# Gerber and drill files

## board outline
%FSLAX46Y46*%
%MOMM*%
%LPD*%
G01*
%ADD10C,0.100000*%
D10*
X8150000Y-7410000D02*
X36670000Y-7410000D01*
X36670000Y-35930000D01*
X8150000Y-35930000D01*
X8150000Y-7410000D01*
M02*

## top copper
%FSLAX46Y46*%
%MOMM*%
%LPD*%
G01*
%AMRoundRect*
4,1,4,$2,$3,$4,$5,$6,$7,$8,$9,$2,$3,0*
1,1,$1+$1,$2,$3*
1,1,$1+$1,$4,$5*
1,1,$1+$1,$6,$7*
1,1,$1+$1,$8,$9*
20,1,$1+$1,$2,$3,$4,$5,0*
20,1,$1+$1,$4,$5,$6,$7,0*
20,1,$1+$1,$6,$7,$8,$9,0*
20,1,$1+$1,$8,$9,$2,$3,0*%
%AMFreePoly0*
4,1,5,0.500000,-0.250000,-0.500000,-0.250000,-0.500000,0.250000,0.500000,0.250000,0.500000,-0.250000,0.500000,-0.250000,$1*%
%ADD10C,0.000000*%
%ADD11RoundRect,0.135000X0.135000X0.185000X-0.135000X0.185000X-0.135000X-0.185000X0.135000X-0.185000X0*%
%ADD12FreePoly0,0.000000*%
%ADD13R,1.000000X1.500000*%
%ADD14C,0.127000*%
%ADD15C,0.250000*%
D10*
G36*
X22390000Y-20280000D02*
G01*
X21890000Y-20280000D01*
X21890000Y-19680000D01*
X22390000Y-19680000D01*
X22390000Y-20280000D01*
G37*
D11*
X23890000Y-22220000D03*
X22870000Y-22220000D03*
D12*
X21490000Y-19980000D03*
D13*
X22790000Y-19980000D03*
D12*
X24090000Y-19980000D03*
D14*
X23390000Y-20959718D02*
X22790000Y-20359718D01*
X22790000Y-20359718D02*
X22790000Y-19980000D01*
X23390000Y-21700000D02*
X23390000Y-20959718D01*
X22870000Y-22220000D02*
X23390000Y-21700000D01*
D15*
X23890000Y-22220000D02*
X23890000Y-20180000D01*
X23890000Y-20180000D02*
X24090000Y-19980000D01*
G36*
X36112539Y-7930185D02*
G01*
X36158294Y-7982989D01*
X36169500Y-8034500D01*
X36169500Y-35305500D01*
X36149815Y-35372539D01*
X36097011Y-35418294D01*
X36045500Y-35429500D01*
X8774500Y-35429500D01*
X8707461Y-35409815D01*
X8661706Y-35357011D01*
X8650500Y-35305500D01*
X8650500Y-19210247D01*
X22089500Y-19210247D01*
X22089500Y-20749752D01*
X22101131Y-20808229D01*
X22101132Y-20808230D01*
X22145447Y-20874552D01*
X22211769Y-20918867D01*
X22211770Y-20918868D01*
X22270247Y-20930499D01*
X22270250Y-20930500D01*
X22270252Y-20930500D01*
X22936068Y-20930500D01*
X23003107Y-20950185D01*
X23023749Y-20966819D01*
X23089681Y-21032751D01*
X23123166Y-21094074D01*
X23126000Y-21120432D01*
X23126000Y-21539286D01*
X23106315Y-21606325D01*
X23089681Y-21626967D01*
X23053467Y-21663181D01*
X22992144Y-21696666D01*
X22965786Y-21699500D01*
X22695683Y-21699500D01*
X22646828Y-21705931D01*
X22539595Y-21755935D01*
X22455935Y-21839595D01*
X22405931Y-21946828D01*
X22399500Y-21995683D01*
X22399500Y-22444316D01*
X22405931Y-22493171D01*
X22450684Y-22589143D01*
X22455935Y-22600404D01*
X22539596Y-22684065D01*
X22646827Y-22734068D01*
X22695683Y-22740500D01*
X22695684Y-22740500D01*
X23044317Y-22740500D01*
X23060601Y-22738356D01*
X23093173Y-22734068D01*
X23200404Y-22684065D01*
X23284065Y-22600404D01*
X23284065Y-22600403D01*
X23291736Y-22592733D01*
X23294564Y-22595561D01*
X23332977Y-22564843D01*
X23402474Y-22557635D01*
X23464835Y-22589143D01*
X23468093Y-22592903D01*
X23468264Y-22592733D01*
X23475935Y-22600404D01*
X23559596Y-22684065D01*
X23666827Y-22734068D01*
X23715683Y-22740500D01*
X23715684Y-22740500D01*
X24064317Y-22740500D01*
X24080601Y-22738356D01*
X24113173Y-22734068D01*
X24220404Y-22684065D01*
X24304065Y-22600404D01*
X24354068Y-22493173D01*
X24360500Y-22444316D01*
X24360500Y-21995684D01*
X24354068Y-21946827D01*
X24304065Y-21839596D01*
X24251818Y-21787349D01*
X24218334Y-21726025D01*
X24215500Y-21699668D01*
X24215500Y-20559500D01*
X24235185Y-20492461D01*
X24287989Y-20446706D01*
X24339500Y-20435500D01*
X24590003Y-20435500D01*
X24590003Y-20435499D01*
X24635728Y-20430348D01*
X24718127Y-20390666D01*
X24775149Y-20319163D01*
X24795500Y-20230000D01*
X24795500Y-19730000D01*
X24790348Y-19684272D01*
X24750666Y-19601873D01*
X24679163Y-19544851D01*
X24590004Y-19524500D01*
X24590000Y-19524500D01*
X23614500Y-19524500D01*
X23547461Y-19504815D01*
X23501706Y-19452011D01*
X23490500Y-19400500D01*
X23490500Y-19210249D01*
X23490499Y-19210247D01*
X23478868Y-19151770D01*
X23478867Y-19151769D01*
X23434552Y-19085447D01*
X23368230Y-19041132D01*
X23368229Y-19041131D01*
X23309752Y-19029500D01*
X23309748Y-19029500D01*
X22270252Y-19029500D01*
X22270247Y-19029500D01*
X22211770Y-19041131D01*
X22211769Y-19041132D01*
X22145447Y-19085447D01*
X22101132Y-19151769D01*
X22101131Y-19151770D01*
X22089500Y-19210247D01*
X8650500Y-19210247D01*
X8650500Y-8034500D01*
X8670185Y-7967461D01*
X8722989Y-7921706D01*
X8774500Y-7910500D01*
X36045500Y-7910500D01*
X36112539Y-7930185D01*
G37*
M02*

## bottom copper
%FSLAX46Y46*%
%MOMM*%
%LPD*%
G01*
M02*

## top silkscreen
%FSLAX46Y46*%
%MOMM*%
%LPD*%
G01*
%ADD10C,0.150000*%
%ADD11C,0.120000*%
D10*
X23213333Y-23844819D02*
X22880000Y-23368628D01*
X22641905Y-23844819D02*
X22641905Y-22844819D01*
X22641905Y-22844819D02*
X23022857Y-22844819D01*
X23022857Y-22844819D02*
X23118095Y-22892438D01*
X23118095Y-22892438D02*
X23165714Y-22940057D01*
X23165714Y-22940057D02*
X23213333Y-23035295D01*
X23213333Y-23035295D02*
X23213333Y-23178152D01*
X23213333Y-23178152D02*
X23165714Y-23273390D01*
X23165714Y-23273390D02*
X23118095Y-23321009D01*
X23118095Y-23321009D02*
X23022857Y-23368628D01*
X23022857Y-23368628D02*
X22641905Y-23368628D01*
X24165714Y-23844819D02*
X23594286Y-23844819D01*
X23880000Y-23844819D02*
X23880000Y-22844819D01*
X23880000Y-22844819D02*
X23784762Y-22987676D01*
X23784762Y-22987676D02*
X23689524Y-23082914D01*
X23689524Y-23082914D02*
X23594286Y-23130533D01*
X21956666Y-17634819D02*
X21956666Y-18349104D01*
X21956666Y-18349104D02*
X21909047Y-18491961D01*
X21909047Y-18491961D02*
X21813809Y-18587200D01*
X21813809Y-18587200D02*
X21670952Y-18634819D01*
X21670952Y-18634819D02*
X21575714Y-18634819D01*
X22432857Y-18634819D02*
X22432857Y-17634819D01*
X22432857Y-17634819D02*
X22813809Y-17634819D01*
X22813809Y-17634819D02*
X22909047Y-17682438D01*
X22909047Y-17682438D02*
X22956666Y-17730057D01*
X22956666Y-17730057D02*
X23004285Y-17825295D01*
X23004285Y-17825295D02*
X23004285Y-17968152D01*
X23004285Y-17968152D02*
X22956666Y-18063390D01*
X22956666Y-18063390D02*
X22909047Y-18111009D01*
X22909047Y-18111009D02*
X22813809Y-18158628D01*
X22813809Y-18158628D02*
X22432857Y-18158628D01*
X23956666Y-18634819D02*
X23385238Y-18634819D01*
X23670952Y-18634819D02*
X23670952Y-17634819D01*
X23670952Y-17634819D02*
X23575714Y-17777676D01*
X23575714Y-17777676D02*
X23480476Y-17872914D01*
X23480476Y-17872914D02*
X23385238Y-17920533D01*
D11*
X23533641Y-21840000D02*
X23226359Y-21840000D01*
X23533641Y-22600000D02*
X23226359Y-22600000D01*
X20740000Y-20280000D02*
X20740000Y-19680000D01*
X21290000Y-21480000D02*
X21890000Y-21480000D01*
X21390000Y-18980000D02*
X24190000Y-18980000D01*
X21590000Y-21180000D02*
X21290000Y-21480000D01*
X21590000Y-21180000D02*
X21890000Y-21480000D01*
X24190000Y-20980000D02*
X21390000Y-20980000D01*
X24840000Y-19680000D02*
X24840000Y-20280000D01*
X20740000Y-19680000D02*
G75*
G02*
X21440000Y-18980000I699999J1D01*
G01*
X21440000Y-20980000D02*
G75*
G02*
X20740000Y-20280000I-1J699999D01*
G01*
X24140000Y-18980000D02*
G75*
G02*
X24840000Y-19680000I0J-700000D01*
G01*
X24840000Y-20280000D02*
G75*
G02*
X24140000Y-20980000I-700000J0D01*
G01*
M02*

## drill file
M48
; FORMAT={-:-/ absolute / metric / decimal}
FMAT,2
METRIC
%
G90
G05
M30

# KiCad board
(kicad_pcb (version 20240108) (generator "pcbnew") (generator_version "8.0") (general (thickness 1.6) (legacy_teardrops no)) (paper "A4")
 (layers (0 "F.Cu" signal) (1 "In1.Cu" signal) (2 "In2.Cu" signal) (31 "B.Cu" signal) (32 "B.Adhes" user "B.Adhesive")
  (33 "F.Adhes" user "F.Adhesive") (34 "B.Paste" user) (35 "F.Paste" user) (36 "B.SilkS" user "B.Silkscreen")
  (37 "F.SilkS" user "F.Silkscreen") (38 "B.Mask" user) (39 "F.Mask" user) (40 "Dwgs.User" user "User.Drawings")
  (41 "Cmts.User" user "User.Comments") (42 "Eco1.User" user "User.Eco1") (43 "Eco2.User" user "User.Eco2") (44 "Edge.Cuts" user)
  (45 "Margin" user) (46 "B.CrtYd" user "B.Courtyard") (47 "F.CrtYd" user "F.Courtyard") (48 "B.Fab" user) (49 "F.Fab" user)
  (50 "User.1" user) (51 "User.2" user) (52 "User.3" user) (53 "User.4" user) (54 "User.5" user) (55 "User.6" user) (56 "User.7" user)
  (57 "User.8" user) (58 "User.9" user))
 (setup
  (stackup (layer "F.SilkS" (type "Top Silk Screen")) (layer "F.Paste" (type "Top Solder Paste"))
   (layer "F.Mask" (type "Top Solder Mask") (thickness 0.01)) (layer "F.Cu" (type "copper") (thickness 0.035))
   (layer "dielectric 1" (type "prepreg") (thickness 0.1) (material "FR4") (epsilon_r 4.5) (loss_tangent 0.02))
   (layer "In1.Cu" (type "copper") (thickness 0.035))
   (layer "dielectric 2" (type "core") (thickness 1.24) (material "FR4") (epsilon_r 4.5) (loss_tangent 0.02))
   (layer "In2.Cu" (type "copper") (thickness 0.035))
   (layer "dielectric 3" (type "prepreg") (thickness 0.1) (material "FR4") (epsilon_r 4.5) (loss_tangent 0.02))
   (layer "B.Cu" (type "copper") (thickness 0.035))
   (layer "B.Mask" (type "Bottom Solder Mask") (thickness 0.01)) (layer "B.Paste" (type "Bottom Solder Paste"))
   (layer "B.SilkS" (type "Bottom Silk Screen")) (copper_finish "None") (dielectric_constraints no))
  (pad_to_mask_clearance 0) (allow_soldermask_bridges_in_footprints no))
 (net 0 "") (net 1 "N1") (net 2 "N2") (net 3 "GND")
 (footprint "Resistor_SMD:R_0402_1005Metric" (layer "F.Cu") (at 23.38 22.22 180)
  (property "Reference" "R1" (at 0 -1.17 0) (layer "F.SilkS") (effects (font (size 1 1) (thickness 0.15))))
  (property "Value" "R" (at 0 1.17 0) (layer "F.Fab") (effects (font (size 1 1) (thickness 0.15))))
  (fp_line (start -0.153641 0.38) (end 0.153641 0.38) (stroke (width 0.12) (type solid)) (layer "F.SilkS"))
  (fp_line (start -0.153641 -0.38) (end 0.153641 -0.38) (stroke (width 0.12) (type solid)) (layer "F.SilkS"))
  (pad "1" smd roundrect (at -0.51 0 180) (size 0.54 0.64) (layers "F.Cu" "F.Paste" "F.Mask") (roundrect_rratio 0.25) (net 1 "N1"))
  (pad "2" smd roundrect (at 0.51 0 180) (size 0.54 0.64) (layers "F.Cu" "F.Paste" "F.Mask") (roundrect_rratio 0.25) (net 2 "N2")))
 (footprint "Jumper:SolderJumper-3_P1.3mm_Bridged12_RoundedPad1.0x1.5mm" (layer "F.Cu") (at 22.79 19.98)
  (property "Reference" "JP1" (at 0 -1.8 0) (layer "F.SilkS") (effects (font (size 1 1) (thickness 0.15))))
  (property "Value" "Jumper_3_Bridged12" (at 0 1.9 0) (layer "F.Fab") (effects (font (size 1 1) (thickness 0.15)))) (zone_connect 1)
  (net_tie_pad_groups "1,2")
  (fp_poly (pts (xy -0.9 -0.3) (xy -0.4 -0.3) (xy -0.4 0.3) (xy -0.9 0.3)) (stroke (width 0) (type solid)) (fill solid) (layer "F.Cu"))
  (fp_line (start -2.05 0.3) (end -2.05 -0.3) (stroke (width 0.12) (type solid)) (layer "F.SilkS"))
  (fp_line (start -1.5 1.5) (end -0.9 1.5) (stroke (width 0.12) (type solid)) (layer "F.SilkS"))
  (fp_line (start -1.4 -1) (end 1.4 -1) (stroke (width 0.12) (type solid)) (layer "F.SilkS"))
  (fp_line (start -1.2 1.2) (end -1.5 1.5) (stroke (width 0.12) (type solid)) (layer "F.SilkS"))
  (fp_line (start -1.2 1.2) (end -0.9 1.5) (stroke (width 0.12) (type solid)) (layer "F.SilkS"))
  (fp_line (start 1.4 1) (end -1.4 1) (stroke (width 0.12) (type solid)) (layer "F.SilkS"))
  (fp_line (start 2.05 -0.3) (end 2.05 0.3) (stroke (width 0.12) (type solid)) (layer "F.SilkS"))
  (fp_arc (start -2.05 -0.3) (mid -1.844975 -0.794975) (end -1.35 -1) (stroke (width 0.12) (type solid)) (layer "F.SilkS"))
  (fp_arc (start -1.35 1) (mid -1.844975 0.794975) (end -2.05 0.3) (stroke (width 0.12) (type solid)) (layer "F.SilkS"))
  (fp_arc (start 1.35 -1) (mid 1.844975 -0.794975) (end 2.05 -0.3) (stroke (width 0.12) (type solid)) (layer "F.SilkS"))
  (fp_arc (start 2.05 0.3) (mid 1.844975 0.794975) (end 1.35 1) (stroke (width 0.12) (type solid)) (layer "F.SilkS"))
  (pad "1" smd custom (at -1.3 0) (size 1 0.5) (layers "F.Cu" "F.Mask") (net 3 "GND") (zone_connect 2) (thermal_bridge_angle 45)
   (options (clearance outline) (anchor rect)) (primitives))
  (pad "2" smd rect (at 0 0) (size 1 1.5) (layers "F.Cu" "F.Mask") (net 2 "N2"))
  (pad "3" smd custom (at 1.3 0) (size 1 0.5) (layers "F.Cu" "F.Mask") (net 1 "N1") (zone_connect 2) (thermal_bridge_angle 45)
   (options (clearance outline) (anchor rect)) (primitives)))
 (gr_rect (start 8.15 7.41) (end 36.67 35.93) (stroke (width 0.1) (type default)) (fill none) (layer "Edge.Cuts"))
 (segment (start 23.39 20.959718) (end 22.79 20.359718) (width 0.127) (layer "F.Cu") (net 2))
 (segment (start 22.79 20.359718) (end 22.79 19.98) (width 0.127) (layer "F.Cu") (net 2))
 (segment (start 23.39 21.7) (end 23.39 20.959718) (width 0.127) (layer "F.Cu") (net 2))
 (segment (start 22.87 22.22) (end 23.39 21.7) (width 0.127) (layer "F.Cu") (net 2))
 (segment (start 23.89 22.22) (end 23.89 20.18) (width 0.25) (layer "F.Cu") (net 1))
 (segment (start 23.89 20.18) (end 24.09 19.98) (width 0.25) (layer "F.Cu") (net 1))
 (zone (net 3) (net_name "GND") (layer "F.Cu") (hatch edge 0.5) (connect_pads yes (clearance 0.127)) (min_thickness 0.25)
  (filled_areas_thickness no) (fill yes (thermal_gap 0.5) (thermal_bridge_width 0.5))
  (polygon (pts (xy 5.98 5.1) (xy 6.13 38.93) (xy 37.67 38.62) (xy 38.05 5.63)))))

